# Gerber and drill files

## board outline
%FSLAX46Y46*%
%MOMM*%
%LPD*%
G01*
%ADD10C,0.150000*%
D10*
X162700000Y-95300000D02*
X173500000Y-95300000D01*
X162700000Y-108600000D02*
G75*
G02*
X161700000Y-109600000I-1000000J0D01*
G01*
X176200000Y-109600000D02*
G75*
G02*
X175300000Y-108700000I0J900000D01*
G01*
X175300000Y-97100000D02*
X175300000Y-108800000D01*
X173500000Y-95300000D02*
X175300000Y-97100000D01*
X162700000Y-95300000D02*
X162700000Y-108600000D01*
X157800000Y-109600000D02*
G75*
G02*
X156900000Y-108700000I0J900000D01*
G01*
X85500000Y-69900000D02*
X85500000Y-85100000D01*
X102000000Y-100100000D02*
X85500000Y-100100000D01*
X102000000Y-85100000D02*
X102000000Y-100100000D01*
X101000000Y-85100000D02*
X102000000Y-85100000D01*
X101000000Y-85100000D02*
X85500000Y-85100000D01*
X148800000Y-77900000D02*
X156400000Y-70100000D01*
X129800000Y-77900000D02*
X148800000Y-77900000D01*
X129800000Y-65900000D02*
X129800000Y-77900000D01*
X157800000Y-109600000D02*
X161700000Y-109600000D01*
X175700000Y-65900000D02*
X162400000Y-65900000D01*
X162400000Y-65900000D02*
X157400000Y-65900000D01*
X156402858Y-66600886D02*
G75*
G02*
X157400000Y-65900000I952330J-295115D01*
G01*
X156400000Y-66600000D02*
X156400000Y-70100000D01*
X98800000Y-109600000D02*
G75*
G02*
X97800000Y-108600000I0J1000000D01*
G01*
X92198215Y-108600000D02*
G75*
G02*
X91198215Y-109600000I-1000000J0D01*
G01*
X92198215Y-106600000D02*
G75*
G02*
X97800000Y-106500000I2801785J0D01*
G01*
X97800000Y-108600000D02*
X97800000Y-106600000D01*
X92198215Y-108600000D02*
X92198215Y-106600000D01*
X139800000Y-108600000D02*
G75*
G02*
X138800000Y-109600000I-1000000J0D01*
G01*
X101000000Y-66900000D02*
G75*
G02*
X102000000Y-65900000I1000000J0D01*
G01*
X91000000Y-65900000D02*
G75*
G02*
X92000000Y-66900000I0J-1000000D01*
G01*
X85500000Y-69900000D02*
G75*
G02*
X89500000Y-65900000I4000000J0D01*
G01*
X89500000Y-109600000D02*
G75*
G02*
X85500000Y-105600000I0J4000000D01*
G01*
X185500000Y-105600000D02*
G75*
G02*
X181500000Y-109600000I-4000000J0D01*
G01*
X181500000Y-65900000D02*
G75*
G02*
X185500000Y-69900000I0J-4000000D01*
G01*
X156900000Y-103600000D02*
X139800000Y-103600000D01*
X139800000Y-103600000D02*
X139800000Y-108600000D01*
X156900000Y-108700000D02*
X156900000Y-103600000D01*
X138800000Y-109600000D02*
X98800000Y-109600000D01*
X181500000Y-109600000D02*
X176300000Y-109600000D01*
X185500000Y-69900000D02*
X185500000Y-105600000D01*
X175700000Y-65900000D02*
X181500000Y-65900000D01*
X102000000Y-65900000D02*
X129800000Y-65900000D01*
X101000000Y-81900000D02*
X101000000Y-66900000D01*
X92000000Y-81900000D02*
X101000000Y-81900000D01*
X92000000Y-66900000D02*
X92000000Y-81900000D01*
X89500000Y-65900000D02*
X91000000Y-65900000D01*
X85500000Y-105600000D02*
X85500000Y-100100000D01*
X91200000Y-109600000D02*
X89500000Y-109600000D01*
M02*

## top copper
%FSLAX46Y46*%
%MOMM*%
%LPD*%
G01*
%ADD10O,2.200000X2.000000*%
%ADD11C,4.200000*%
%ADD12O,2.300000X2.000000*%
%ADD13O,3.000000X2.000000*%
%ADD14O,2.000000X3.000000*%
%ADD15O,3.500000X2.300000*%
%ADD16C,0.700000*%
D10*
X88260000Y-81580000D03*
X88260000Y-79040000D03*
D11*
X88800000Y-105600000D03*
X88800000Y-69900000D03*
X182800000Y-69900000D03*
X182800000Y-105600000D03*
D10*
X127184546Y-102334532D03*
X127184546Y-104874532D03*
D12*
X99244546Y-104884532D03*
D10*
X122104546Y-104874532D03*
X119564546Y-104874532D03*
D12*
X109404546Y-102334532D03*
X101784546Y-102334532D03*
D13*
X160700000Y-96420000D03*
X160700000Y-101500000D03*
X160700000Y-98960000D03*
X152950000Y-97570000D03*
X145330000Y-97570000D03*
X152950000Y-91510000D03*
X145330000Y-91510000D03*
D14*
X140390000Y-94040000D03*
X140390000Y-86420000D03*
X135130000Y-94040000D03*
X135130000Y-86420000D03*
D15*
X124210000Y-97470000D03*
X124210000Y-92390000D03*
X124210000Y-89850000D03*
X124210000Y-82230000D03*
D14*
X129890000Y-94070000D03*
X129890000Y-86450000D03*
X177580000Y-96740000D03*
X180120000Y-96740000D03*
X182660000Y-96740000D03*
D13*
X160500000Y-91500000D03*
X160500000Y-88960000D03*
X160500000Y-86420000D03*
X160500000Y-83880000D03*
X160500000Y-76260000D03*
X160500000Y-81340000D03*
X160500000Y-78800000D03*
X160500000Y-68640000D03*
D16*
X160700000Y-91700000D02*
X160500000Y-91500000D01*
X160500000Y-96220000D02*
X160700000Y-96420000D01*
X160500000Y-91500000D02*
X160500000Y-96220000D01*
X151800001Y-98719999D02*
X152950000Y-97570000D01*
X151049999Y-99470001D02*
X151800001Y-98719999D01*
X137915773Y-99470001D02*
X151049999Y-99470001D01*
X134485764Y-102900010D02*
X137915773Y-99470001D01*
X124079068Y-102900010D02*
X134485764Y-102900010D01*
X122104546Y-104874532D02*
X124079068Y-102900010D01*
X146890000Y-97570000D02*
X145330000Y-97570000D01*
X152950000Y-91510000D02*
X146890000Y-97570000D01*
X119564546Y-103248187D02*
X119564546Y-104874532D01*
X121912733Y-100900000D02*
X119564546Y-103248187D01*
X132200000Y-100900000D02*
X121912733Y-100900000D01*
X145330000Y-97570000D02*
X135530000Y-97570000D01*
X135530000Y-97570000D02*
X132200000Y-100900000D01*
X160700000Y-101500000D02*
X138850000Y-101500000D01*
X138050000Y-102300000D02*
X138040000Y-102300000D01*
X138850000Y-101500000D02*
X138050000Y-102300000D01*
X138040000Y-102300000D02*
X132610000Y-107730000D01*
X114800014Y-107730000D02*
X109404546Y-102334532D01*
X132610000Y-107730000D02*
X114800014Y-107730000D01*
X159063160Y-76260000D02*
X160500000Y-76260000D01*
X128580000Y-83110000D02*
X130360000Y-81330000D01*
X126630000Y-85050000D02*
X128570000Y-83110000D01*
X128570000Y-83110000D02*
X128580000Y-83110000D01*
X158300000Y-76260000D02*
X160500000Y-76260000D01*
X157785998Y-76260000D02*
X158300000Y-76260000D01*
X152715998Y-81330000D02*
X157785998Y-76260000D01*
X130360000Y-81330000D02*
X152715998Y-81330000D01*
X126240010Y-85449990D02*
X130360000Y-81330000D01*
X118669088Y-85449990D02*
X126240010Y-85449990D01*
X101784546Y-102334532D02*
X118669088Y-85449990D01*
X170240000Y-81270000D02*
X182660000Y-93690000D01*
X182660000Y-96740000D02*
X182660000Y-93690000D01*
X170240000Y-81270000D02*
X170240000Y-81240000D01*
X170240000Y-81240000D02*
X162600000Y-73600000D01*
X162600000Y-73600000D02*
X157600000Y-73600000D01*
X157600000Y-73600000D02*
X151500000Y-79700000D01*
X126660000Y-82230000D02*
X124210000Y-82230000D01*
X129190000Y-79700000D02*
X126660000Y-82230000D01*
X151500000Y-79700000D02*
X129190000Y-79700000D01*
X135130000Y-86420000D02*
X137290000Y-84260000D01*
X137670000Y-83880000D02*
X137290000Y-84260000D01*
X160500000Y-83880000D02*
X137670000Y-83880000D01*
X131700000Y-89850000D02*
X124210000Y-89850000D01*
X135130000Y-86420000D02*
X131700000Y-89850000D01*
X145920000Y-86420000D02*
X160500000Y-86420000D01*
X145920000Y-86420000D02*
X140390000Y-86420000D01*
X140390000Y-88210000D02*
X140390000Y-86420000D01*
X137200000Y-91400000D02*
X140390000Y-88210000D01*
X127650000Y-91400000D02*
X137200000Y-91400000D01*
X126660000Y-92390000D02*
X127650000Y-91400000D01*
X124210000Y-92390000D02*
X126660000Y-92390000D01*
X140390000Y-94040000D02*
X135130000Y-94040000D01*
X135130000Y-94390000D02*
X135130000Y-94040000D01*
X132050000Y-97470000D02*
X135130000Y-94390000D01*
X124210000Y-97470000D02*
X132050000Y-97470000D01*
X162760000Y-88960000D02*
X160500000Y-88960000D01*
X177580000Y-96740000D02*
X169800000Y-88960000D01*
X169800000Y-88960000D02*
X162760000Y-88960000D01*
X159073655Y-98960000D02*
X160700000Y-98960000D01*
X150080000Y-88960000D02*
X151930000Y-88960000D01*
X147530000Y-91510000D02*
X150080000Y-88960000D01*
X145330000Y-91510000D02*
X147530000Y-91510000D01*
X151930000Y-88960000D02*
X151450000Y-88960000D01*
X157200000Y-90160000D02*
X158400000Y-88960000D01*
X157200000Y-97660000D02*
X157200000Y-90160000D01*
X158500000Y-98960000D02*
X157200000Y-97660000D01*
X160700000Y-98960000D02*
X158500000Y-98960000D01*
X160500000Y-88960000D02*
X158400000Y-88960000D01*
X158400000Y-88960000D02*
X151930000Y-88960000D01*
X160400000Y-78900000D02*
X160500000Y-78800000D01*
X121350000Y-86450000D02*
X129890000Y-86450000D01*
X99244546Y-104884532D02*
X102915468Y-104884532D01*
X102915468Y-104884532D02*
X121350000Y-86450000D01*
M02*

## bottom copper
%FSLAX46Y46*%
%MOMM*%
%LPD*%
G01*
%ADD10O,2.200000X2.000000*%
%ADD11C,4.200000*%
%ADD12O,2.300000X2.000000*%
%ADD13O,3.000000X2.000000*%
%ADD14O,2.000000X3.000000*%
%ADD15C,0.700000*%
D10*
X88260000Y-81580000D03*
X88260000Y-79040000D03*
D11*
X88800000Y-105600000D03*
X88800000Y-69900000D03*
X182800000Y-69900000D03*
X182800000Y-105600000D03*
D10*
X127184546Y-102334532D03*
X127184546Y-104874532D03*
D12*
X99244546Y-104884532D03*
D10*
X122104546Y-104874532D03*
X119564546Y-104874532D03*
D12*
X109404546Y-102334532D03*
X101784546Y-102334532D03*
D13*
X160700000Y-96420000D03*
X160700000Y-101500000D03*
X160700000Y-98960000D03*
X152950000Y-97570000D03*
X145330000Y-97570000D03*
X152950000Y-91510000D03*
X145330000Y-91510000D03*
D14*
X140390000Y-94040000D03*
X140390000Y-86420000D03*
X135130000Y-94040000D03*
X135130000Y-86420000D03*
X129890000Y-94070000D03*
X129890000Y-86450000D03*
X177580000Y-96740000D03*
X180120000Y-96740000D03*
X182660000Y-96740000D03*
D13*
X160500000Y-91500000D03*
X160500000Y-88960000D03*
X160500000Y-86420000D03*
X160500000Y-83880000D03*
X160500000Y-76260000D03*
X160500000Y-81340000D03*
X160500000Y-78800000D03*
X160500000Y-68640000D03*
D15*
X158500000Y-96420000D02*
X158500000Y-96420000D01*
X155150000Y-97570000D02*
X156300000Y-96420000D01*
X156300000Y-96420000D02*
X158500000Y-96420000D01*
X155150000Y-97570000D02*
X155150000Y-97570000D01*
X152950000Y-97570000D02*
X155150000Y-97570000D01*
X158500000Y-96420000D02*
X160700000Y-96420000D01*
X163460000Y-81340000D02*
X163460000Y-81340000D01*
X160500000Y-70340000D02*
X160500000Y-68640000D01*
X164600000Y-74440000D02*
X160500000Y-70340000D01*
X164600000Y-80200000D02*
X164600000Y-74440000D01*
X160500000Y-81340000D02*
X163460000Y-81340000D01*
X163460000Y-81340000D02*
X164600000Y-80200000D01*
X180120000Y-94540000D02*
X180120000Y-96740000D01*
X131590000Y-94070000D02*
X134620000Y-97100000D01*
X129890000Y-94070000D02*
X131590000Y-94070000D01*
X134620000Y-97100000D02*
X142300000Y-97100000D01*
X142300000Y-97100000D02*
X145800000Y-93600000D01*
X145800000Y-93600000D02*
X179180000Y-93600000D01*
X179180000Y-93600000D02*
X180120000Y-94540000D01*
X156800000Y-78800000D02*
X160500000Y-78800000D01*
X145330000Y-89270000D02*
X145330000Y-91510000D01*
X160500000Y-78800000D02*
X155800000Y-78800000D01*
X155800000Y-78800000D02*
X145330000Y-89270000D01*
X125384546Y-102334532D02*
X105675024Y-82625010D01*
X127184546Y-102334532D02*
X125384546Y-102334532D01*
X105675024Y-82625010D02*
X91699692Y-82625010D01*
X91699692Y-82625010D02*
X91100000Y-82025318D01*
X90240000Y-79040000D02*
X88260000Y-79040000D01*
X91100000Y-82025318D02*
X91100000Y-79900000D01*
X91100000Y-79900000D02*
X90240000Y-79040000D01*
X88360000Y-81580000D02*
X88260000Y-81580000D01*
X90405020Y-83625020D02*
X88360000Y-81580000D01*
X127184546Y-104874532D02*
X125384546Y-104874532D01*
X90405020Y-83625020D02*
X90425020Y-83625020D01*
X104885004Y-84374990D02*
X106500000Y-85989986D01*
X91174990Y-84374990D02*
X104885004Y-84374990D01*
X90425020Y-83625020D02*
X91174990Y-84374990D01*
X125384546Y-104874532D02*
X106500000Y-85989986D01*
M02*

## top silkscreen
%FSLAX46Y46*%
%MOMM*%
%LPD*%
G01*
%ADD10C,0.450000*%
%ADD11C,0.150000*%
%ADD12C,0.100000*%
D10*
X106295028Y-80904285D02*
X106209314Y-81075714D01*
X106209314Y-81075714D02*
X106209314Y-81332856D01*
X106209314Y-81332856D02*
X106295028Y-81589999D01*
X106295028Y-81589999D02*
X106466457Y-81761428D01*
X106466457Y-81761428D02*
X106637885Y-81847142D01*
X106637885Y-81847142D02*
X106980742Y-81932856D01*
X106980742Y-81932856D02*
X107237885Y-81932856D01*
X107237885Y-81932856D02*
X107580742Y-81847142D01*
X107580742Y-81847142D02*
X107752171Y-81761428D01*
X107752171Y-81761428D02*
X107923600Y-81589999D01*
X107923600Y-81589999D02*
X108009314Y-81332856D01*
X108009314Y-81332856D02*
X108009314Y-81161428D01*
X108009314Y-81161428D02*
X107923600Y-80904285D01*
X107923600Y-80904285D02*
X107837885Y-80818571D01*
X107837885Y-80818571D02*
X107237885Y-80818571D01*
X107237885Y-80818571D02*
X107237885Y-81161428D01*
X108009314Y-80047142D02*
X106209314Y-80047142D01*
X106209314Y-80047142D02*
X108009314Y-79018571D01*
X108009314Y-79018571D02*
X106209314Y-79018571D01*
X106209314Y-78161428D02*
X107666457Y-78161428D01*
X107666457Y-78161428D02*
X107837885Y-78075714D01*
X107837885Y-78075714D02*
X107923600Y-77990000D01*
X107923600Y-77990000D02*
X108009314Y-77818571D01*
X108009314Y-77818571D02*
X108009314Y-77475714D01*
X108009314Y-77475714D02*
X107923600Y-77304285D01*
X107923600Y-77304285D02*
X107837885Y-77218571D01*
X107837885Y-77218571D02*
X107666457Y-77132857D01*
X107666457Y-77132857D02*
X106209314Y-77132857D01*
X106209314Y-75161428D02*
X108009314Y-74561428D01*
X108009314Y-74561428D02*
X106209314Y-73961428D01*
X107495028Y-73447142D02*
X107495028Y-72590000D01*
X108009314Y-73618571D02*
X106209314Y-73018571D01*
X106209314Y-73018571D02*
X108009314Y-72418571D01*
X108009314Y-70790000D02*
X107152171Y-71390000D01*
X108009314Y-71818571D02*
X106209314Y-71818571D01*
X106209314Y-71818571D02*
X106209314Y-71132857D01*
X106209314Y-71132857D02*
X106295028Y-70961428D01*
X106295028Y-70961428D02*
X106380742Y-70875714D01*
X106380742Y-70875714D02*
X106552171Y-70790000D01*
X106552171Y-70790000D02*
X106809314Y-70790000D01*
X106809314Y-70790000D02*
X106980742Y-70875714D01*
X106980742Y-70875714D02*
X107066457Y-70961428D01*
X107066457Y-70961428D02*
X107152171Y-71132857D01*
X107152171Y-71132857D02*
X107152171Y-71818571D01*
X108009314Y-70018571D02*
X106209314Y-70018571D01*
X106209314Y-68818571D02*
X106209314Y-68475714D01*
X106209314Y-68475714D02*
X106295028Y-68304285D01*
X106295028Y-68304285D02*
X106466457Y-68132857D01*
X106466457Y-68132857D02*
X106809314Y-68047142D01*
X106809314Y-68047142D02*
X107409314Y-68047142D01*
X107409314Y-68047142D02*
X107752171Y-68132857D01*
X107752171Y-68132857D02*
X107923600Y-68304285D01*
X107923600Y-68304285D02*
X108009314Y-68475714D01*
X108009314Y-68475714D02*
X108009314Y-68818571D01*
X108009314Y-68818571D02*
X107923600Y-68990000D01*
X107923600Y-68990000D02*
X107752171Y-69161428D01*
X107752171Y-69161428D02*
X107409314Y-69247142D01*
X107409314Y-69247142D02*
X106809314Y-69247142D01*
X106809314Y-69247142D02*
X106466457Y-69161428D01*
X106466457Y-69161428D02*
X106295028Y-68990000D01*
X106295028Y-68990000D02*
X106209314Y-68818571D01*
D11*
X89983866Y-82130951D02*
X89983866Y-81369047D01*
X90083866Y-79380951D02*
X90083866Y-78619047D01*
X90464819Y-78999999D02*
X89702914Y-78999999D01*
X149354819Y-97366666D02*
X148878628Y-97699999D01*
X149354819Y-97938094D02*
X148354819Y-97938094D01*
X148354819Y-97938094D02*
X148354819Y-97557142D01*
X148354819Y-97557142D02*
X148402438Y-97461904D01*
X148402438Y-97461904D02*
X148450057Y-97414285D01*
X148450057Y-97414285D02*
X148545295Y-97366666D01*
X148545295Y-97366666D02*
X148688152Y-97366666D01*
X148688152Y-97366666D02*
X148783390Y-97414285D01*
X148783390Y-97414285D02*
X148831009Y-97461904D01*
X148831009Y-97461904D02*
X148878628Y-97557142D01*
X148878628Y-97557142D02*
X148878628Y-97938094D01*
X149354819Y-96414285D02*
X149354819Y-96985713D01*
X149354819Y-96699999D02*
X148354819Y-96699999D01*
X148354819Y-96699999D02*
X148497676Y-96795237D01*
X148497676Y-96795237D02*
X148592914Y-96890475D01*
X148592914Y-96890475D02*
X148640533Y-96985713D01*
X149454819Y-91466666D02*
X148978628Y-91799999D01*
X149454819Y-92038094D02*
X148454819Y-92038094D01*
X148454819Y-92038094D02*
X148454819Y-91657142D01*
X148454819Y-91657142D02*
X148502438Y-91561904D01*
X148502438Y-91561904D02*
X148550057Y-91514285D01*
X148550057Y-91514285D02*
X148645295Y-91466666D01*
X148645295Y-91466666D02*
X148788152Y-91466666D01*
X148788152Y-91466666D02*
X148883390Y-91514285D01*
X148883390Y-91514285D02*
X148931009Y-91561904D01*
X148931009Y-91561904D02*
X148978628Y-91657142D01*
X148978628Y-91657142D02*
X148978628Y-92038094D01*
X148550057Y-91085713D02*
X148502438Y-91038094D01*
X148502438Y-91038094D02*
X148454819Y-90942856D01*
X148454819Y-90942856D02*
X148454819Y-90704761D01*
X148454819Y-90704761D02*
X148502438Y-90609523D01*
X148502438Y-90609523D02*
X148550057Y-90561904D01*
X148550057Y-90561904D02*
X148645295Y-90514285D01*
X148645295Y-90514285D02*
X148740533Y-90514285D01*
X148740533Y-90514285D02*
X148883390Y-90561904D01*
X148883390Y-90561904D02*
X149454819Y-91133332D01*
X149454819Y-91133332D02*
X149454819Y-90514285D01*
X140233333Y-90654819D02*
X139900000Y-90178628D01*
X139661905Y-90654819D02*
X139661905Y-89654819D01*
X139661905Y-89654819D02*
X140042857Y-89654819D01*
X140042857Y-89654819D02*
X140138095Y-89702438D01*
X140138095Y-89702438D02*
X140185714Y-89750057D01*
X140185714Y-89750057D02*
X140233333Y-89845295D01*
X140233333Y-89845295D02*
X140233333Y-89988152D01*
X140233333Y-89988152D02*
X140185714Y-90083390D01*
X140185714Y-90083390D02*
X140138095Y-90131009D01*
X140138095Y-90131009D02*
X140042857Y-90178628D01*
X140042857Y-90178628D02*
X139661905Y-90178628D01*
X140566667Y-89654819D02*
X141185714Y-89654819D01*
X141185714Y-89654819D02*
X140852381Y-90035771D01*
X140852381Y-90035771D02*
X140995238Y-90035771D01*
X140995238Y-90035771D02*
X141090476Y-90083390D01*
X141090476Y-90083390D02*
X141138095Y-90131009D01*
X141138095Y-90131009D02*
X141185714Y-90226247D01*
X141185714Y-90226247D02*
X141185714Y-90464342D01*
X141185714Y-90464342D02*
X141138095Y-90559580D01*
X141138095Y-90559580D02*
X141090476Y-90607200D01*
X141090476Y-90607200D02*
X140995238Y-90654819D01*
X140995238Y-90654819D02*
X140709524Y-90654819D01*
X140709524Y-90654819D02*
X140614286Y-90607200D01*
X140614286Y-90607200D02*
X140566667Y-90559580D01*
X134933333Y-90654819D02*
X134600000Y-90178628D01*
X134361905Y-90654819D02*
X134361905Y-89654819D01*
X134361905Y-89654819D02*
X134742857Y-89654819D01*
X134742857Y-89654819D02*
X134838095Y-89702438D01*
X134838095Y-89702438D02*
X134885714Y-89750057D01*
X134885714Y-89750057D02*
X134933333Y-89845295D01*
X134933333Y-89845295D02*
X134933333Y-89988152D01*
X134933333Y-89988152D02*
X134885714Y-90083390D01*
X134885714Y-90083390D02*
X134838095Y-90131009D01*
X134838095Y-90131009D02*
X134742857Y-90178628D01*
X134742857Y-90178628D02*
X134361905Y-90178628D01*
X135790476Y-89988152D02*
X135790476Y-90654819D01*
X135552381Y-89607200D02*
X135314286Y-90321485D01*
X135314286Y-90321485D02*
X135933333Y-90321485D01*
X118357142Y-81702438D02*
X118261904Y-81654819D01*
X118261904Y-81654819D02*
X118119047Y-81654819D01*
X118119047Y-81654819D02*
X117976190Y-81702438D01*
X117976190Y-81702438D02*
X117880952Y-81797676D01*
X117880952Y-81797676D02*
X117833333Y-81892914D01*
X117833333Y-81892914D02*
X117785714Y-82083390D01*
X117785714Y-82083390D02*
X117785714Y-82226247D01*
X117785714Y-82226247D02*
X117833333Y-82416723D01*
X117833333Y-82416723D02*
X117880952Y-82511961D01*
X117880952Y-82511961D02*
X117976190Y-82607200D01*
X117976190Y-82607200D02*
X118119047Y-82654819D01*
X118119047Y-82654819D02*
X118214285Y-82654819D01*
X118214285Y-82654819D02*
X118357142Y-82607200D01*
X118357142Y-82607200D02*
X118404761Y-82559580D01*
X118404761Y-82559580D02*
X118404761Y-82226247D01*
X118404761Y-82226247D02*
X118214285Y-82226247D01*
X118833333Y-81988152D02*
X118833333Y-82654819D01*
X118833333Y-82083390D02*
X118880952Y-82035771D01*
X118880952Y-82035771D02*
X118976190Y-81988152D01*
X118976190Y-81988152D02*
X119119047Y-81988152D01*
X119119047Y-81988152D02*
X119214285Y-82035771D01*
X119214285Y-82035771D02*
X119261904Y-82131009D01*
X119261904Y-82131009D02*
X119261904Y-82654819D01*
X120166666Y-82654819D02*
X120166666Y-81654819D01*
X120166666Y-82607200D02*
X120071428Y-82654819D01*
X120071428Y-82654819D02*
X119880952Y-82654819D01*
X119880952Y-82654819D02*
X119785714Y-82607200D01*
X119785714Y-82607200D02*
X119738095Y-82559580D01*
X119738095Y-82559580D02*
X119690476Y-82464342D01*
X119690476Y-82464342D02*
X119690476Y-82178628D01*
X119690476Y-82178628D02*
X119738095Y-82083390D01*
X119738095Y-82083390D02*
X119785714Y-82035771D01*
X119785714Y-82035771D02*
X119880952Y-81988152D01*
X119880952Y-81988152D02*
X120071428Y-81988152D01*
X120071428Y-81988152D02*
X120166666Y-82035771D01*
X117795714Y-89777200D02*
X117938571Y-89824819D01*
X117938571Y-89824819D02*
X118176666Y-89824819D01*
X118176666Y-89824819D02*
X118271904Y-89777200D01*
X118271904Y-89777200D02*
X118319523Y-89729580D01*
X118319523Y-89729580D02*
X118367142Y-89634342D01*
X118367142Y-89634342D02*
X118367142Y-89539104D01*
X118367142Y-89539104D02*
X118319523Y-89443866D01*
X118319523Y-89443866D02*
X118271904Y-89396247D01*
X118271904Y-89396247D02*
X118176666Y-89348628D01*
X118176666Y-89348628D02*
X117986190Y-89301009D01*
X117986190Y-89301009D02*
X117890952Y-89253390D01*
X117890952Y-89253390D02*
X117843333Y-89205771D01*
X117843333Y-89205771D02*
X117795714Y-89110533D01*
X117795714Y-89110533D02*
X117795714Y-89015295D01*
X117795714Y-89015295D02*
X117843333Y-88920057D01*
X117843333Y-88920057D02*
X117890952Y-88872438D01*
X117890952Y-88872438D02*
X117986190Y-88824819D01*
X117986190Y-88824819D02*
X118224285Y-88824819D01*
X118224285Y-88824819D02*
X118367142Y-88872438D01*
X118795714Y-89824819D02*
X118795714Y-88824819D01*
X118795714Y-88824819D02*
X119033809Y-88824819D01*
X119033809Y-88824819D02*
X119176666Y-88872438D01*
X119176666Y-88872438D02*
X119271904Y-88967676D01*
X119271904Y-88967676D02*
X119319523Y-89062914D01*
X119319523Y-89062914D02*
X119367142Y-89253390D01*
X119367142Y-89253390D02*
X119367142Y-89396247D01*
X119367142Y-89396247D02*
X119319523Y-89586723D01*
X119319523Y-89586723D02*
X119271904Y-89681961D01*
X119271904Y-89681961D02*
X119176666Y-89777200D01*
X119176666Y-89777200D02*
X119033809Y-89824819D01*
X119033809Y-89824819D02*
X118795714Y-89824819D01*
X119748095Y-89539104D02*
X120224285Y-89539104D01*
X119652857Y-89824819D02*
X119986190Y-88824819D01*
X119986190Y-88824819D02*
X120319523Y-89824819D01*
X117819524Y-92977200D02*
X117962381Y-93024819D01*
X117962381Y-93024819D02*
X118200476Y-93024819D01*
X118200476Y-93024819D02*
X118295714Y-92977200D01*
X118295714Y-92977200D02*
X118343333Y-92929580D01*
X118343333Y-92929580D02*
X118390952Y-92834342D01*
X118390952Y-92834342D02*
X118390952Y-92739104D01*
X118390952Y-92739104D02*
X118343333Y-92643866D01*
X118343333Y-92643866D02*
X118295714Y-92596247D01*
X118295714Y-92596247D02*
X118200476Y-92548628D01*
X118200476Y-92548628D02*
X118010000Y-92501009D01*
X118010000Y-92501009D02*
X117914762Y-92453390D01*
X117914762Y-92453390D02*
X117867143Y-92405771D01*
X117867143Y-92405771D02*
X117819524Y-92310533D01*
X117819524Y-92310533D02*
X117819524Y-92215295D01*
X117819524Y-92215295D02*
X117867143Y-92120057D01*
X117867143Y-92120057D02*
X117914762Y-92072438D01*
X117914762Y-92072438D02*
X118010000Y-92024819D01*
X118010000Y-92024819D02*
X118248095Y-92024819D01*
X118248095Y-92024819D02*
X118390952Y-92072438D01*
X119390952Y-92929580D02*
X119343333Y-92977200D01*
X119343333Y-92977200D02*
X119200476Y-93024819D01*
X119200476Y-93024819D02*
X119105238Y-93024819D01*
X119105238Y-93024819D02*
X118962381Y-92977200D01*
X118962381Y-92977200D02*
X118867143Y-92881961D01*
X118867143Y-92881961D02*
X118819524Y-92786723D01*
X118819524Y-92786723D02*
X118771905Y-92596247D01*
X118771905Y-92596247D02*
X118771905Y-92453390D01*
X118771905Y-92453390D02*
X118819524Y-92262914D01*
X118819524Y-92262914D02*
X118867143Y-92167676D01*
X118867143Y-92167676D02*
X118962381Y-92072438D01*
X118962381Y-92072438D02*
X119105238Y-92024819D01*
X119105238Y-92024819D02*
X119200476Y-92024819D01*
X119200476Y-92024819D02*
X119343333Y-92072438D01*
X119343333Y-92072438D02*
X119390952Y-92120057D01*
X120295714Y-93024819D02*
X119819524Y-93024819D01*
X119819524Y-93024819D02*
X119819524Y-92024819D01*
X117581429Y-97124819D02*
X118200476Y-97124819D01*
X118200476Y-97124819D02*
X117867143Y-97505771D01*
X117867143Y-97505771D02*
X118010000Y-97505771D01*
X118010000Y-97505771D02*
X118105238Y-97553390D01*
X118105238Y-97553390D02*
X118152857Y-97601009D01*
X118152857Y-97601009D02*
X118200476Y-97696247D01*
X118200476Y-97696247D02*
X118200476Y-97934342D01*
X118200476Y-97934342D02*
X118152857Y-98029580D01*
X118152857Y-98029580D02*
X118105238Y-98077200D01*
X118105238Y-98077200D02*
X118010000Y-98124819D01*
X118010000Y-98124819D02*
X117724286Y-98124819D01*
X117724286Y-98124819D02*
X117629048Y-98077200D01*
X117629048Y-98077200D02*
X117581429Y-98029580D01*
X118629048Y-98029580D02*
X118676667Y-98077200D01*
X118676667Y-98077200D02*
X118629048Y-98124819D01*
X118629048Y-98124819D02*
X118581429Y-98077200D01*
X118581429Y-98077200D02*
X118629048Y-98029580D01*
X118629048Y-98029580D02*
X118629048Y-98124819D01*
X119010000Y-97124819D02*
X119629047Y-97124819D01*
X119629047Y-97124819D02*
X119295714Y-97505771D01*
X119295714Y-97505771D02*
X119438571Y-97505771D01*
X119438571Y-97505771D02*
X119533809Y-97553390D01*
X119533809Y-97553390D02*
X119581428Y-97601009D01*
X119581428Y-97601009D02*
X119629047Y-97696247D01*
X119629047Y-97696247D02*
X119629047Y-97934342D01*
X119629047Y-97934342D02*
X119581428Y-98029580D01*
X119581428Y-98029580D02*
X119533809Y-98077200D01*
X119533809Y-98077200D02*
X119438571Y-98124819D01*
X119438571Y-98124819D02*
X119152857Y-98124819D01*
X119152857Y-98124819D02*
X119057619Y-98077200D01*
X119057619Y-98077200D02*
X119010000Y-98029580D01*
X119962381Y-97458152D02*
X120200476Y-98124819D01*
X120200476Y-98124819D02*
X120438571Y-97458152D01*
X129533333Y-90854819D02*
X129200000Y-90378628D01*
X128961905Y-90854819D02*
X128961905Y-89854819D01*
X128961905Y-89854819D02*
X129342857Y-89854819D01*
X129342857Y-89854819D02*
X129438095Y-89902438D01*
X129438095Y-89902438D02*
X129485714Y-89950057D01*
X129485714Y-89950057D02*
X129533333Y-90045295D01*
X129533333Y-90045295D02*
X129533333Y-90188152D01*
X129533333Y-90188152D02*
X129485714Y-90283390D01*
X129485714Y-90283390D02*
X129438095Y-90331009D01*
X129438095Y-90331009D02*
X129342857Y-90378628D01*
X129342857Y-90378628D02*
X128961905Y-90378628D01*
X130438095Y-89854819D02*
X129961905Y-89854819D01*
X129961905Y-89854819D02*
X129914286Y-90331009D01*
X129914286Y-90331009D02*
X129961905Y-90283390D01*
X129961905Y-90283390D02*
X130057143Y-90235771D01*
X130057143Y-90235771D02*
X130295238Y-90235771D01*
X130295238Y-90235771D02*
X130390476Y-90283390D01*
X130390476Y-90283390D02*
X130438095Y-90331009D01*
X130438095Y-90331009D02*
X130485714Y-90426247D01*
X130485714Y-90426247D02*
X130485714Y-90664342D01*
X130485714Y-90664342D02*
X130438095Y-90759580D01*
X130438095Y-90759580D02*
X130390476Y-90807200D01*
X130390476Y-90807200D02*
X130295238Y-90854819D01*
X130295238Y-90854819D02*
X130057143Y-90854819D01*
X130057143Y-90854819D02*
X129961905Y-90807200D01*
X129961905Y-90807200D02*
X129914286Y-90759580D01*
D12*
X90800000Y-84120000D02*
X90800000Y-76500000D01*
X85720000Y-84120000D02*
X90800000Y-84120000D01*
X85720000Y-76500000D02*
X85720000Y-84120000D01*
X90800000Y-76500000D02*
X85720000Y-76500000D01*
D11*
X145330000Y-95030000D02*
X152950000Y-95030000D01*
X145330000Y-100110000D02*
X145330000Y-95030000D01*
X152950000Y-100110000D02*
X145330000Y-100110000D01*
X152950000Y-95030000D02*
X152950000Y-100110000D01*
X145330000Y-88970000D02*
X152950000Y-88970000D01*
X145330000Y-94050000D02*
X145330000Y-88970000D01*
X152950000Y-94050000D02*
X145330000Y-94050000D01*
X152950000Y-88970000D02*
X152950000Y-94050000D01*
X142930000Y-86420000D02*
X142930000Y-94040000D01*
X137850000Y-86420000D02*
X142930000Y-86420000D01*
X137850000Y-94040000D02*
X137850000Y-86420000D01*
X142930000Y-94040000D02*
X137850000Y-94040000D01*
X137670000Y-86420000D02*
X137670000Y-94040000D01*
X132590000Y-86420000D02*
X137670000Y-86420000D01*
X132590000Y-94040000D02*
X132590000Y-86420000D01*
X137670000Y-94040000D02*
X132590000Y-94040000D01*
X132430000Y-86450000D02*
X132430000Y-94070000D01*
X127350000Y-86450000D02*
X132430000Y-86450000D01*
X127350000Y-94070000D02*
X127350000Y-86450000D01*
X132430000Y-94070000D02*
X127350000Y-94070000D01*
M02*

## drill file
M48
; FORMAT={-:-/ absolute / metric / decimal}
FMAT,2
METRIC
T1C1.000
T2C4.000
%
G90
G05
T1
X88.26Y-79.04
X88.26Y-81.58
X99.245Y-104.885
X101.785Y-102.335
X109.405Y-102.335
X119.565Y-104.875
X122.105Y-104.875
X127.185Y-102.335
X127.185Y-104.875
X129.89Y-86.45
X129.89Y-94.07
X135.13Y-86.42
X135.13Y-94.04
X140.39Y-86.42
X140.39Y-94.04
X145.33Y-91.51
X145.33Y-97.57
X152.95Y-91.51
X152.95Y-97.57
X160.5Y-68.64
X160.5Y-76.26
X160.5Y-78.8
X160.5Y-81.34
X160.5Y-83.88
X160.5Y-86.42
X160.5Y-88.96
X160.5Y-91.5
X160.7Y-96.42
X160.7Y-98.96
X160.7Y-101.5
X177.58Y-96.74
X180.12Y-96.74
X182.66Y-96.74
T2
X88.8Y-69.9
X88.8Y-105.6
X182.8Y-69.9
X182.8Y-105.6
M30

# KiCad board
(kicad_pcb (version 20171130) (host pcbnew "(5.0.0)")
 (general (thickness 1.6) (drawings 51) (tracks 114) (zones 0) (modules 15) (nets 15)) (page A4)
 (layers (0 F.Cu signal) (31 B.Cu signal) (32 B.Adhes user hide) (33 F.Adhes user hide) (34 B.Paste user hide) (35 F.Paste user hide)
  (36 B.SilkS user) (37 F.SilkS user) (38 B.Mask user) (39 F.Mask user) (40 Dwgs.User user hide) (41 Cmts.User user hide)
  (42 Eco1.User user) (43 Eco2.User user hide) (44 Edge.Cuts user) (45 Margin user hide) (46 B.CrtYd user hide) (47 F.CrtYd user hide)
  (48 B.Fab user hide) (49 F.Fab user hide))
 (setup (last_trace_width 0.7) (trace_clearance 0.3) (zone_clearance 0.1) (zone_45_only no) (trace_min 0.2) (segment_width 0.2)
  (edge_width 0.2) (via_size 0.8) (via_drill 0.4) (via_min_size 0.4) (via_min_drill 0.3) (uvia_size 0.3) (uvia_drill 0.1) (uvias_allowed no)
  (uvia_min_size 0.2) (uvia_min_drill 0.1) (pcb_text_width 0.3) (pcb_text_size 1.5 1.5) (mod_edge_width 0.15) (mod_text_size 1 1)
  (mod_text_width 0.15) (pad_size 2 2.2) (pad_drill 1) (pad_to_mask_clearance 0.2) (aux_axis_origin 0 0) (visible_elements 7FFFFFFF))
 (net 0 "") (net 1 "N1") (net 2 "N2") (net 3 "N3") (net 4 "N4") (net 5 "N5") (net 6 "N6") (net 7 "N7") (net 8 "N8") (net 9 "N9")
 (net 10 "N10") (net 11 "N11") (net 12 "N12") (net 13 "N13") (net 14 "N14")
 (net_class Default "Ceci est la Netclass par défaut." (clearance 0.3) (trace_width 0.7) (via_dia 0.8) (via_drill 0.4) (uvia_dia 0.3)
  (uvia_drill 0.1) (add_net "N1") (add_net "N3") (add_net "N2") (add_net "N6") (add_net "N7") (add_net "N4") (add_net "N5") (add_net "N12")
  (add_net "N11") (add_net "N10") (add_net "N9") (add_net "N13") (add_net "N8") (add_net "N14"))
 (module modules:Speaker (layer B.Cu) (at 90.8 76.5 270)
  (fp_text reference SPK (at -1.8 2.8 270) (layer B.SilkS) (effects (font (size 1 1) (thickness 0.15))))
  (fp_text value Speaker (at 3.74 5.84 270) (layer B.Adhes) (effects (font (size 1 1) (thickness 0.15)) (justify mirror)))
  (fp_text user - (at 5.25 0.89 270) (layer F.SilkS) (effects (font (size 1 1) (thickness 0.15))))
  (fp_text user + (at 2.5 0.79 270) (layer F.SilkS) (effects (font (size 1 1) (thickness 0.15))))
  (fp_line (start 7.62 0) (end 0 0) (layer F.SilkS) (width 0.1))
  (fp_line (start 7.62 5.08) (end 7.62 0) (layer F.SilkS) (width 0.1))
  (fp_line (start 0 5.08) (end 7.62 5.08) (layer F.SilkS) (width 0.1))
  (fp_line (start 0 0) (end 0 5.08) (layer F.SilkS) (width 0.1))
  (pad 2 thru_hole oval (at 5.08 2.54 270) (size 2 2.2) (drill 1) (layers *.Cu *.Paste *.Mask) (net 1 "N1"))
  (pad 1 thru_hole oval (at 2.54 2.54 270) (size 2 2.2) (drill 1) (layers *.Cu *.Paste *.Mask) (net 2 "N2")))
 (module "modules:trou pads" (layer F.Cu) (at 88.8 105.6)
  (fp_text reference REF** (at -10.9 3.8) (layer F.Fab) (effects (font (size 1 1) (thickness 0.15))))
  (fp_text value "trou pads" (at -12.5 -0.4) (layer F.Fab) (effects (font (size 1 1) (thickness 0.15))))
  (pad "" np_thru_hole circle (at 0 0) (size 4.2 4.2) (drill 4) (layers *.Cu *.Mask)))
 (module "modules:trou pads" (layer F.Cu) (at 88.8 69.9)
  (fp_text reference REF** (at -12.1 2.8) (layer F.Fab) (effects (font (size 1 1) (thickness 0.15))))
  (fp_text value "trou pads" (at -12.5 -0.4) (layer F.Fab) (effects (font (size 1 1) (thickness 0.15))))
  (pad "" np_thru_hole circle (at 0 0) (size 4.2 4.2) (drill 4) (layers *.Cu *.Mask)))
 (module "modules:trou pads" (layer F.Cu) (at 182.8 69.9)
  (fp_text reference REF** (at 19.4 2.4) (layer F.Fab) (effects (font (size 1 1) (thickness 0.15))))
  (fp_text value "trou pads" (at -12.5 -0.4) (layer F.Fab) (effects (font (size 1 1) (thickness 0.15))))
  (pad "" np_thru_hole circle (at 0 0) (size 4.2 4.2) (drill 4) (layers *.Cu *.Mask)))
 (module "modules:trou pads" (layer F.Cu) (at 182.8 105.6)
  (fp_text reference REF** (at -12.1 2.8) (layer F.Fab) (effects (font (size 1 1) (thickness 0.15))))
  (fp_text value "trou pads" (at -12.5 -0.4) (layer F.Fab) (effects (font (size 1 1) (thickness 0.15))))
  (pad "" np_thru_hole circle (at 0 0) (size 4.2 4.2) (drill 4) (layers *.Cu *.Mask)))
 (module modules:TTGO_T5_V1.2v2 (layer F.Cu) (at 127.734546 102.554532 90)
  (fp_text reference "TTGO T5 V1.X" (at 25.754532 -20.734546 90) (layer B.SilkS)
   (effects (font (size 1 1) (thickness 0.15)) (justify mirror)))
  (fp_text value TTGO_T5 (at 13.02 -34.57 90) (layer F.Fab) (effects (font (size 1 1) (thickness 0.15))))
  (pad "HP +" thru_hole oval (at 0.22 -0.55 90) (size 2 2.2) (drill 1) (layers *.Cu *.Paste *.Mask) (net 2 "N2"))
  (pad "HP -" thru_hole oval (at -2.32 -0.55 90) (size 2 2.2) (drill 1) (layers *.Cu *.Paste *.Mask) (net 1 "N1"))
  (pad 12 thru_hole oval (at -2.33 -28.49 90) (size 2 2.3) (drill 1) (layers *.Cu *.Paste *.Mask) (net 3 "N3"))
  (pad 3 thru_hole oval (at -2.32 -5.63 90) (size 2 2.2) (drill 1) (layers *.Cu *.Paste *.Mask) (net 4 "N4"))
  (pad 4 thru_hole oval (at -2.32 -8.17 90) (size 2 2.2) (drill 1) (layers *.Cu *.Paste *.Mask) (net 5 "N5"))
  (pad 20 thru_hole oval (at 0.22 -18.33 90) (size 2 2.3) (drill 1) (layers *.Cu *.Paste *.Mask) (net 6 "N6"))
  (pad 23 thru_hole oval (at 0.22 -25.95 90) (size 2 2.3) (drill 1) (layers *.Cu *.Paste *.Mask) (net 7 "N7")))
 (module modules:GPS (layer F.Cu) (at 160.7 96.42 270)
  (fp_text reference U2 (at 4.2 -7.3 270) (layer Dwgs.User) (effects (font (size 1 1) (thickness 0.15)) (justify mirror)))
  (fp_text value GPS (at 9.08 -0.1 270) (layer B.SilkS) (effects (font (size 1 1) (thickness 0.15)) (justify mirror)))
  (pad 1 thru_hole oval (at 0 0 270) (size 2 3) (drill 1) (layers *.Cu *.Paste *.Mask) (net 4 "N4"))
  (pad 3 thru_hole oval (at 5.08 0 270) (size 2 3) (drill 1) (layers *.Cu *.Paste *.Mask) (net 6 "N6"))
  (pad 2 thru_hole oval (at 2.54 0 270) (size 2 3) (drill 1) (layers *.Cu *.Paste *.Mask) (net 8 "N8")))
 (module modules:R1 (layer F.Cu) (at 145.33 97.57 270)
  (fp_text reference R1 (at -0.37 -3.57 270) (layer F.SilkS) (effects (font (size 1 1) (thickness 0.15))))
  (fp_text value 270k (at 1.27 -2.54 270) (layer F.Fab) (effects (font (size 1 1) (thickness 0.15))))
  (fp_line (start -2.54 0) (end -2.54 -7.62) (layer F.SilkS) (width 0.15))
  (fp_line (start 2.54 0) (end -2.54 0) (layer F.SilkS) (width 0.15))
  (fp_line (start 2.54 -7.62) (end 2.54 0) (layer F.SilkS) (width 0.15))
  (fp_line (start -2.54 -7.62) (end 2.54 -7.62) (layer F.SilkS) (width 0.15))
  (pad 2 thru_hole oval (at 0 -7.62 270) (size 2 3) (drill 1) (layers *.Cu *.Paste *.Mask) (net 4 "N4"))
  (pad 1 thru_hole oval (at 0 0 270) (size 2 3) (drill 1) (layers *.Cu *.Paste *.Mask) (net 5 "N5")))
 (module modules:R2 (layer F.Cu) (at 145.33 91.51 270)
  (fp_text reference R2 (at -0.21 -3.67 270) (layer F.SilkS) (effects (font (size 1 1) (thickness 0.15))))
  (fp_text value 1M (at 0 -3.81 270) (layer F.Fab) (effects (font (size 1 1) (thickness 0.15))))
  (fp_line (start -2.54 0) (end -2.54 -7.62) (layer F.SilkS) (width 0.15))
  (fp_line (start 2.54 0) (end -2.54 0) (layer F.SilkS) (width 0.15))
  (fp_line (start 2.54 -7.62) (end 2.54 0) (layer F.SilkS) (width 0.15))
  (fp_line (start -2.54 -7.62) (end 2.54 -7.62) (layer F.SilkS) (width 0.15))
  (pad 2 thru_hole oval (at 0 -7.62 270) (size 2 3) (drill 1) (layers *.Cu *.Paste *.Mask) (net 5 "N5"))
  (pad 1 thru_hole oval (at 0 0 270) (size 2 3) (drill 1) (layers *.Cu *.Paste *.Mask) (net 8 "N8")))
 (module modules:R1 (layer F.Cu) (at 140.39 86.42 180)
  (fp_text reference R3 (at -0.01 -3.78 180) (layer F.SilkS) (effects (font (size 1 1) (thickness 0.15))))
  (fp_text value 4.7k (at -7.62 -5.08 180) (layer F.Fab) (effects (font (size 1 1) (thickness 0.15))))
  (fp_line (start -2.54 0) (end -2.54 -7.62) (layer F.SilkS) (width 0.15))
  (fp_line (start 2.54 0) (end -2.54 0) (layer F.SilkS) (width 0.15))
  (fp_line (start 2.54 -7.62) (end 2.54 0) (layer F.SilkS) (width 0.15))
  (fp_line (start -2.54 -7.62) (end 2.54 -7.62) (layer F.SilkS) (width 0.15))
  (pad 2 thru_hole oval (at 0 -7.62 180) (size 2 3) (drill 1) (layers *.Cu *.Paste *.Mask) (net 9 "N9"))
  (pad 1 thru_hole oval (at 0 0 180) (size 2 3) (drill 1) (layers *.Cu *.Paste *.Mask) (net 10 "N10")))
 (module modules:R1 (layer F.Cu) (at 135.13 86.42 180)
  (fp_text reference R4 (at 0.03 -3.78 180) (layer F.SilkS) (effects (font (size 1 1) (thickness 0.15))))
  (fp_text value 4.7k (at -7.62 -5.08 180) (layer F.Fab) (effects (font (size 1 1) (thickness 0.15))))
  (fp_line (start -2.54 0) (end -2.54 -7.62) (layer F.SilkS) (width 0.15))
  (fp_line (start 2.54 0) (end -2.54 0) (layer F.SilkS) (width 0.15))
  (fp_line (start 2.54 -7.62) (end 2.54 0) (layer F.SilkS) (width 0.15))
  (fp_line (start -2.54 -7.62) (end 2.54 -7.62) (layer F.SilkS) (width 0.15))
  (pad 2 thru_hole oval (at 0 -7.62 180) (size 2 3) (drill 1) (layers *.Cu *.Paste *.Mask) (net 9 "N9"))
  (pad 1 thru_hole oval (at 0 0 180) (size 2 3) (drill 1) (layers *.Cu *.Paste *.Mask) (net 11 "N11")))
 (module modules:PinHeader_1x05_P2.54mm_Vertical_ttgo (layer F.Cu) (at 124.21 84.77)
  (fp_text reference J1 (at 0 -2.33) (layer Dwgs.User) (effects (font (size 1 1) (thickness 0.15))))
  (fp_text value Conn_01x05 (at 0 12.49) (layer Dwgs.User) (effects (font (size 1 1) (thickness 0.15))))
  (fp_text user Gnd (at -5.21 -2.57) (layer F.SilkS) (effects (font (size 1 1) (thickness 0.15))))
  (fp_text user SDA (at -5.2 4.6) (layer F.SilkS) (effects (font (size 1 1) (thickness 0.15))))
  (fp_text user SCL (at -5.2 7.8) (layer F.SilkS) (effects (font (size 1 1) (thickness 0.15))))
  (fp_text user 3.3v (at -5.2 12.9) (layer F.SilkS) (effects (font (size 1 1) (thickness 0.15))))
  (pad 5 smd oval (at 0 12.7) (size 3.5 2.3) (layers F.Cu F.Paste F.Mask) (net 9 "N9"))
  (pad 4 smd oval (at 0 7.62) (size 3.5 2.3) (layers F.Cu F.Paste F.Mask) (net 10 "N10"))
  (pad 3 smd oval (at 0 5.08) (size 3.5 2.3) (layers F.Cu F.Paste F.Mask) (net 11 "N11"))
  (pad 1 smd oval (at 0 -2.54) (size 3.5 2.3) (layers F.Cu F.Paste F.Mask) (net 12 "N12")))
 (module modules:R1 (layer F.Cu) (at 129.89 86.45 180)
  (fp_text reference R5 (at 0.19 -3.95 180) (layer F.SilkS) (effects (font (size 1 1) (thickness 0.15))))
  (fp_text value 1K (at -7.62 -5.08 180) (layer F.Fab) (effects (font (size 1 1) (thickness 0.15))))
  (fp_line (start -2.54 0) (end -2.54 -7.62) (layer F.SilkS) (width 0.15))
  (fp_line (start 2.54 0) (end -2.54 0) (layer F.SilkS) (width 0.15))
  (fp_line (start 2.54 -7.62) (end 2.54 0) (layer F.SilkS) (width 0.15))
  (fp_line (start -2.54 -7.62) (end 2.54 -7.62) (layer F.SilkS) (width 0.15))
  (pad 2 thru_hole oval (at 0 -7.62 180) (size 2 3) (drill 1) (layers *.Cu *.Paste *.Mask) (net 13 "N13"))
  (pad 1 thru_hole oval (at 0 0 180) (size 2 3) (drill 1) (layers *.Cu *.Paste *.Mask) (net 3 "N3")))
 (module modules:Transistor (layer F.Cu) (at 185.2 94.2 180)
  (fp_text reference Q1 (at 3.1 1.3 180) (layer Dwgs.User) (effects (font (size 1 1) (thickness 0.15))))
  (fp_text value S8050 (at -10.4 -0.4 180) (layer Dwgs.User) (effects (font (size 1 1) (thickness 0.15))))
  (pad 3 thru_hole oval (at 7.62 -2.54 180) (size 2 3) (drill 1) (layers *.Cu *.Paste *.Mask) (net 8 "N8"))
  (pad 2 thru_hole oval (at 5.08 -2.54 180) (size 2 3) (drill 1) (layers *.Cu *.Paste *.Mask) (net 13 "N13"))
  (pad 1 thru_hole oval (at 2.54 -2.54 180) (size 2 3) (drill 1) (layers *.Cu *.Paste *.Mask) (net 12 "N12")))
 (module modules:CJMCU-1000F (layer B.Cu) (at 163.04 78.8 270)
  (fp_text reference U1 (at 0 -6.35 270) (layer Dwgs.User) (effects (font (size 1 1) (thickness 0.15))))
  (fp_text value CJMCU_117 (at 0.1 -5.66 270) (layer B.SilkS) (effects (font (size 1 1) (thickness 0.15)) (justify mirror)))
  (pad 1 thru_hole oval (at 12.7 2.54 270) (size 2 3) (drill 1) (layers *.Cu *.Paste *.Mask) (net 4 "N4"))
  (pad 2 thru_hole oval (at 10.16 2.54 270) (size 2 3) (drill 1) (layers *.Cu *.Paste *.Mask) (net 8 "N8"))
  (pad 3 thru_hole oval (at 7.62 2.54 270) (size 2 3) (drill 1) (layers *.Cu *.Paste *.Mask) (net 10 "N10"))
  (pad 4 thru_hole oval (at 5.08 2.54 270) (size 2 3) (drill 1) (layers *.Cu *.Paste *.Mask) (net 11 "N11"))
  (pad 7 thru_hole oval (at -2.54 2.54 270) (size 2 3) (drill 1) (layers *.Cu *.Paste *.Mask) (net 7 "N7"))
  (pad 5 thru_hole oval (at 2.54 2.54 270) (size 2 3) (drill 1) (layers *.Cu *.Paste *.Mask) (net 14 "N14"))
  (pad 6 thru_hole oval (at 0 2.54 270) (size 2 3) (drill 1) (layers *.Cu *.Paste *.Mask) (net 8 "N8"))
  (pad 10 thru_hole oval (at -10.16 2.54 270) (size 2 3) (drill 1) (layers *.Cu *.Paste *.Mask) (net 14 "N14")))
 (gr_line (start 162.7 95.3) (end 173.5 95.3) (layer Edge.Cuts) (width 0.15))
 (gr_arc (start 161.7 108.6) (end 161.7 109.6) (angle -90) (layer Edge.Cuts) (width 0.15))
 (gr_arc (start 176.2 108.7) (end 175.3 108.7) (angle -90) (layer Edge.Cuts) (width 0.15))
 (gr_line (start 175.3 97.1) (end 175.3 108.8) (layer Edge.Cuts) (width 0.15))
 (gr_line (start 173.5 95.3) (end 175.3 97.1) (layer Edge.Cuts) (width 0.15))
 (gr_line (start 162.7 95.3) (end 162.7 108.6) (layer Edge.Cuts) (width 0.15))
 (gr_arc (start 157.8 108.7) (end 156.9 108.7) (angle -90) (layer Edge.Cuts) (width 0.15))
 (gr_line (start 85.5 69.9) (end 85.5 85.1) (layer Edge.Cuts) (width 0.15))
 (gr_line (start 102 100.1) (end 85.5 100.1) (layer Edge.Cuts) (width 0.15))
 (gr_line (start 102 85.1) (end 102 100.1) (layer Edge.Cuts) (width 0.15))
 (gr_line (start 101 85.1) (end 102 85.1) (layer Edge.Cuts) (width 0.15))
 (gr_line (start 101 85.1) (end 85.5 85.1) (layer Edge.Cuts) (width 0.15))
 (gr_line (start 148.8 77.9) (end 156.4 70.1) (layer Edge.Cuts) (width 0.15))
 (gr_line (start 129.8 77.9) (end 148.8 77.9) (layer Edge.Cuts) (width 0.15))
 (gr_line (start 129.8 65.9) (end 129.8 77.9) (layer Edge.Cuts) (width 0.15))
 (gr_line (start 157.8 109.6) (end 161.7 109.6) (layer Edge.Cuts) (width 0.15))
 (gr_line (start 175.7 65.9) (end 162.4 65.9) (layer Edge.Cuts) (width 0.15))
 (gr_line (start 162.4 65.9) (end 157.4 65.9) (layer Edge.Cuts) (width 0.15))
 (gr_arc (start 157.355188 66.896001) (end 157.4 65.9) (angle -75.35856355) (layer Edge.Cuts) (width 0.15))
 (gr_line (start 156.4 66.6) (end 156.4 70.1) (layer Edge.Cuts) (width 0.15))
 (gr_arc (start 98.8 108.6) (end 97.8 108.6) (angle -90) (layer Edge.Cuts) (width 0.15))
 (gr_arc (start 91.198215 108.6) (end 91.198215 109.6) (angle -90) (layer Edge.Cuts) (width 0.15))
 (gr_arc (start 95 106.6) (end 97.8 106.5) (angle -177.9545915) (layer Edge.Cuts) (width 0.15))
 (gr_line (start 97.8 108.6) (end 97.8 106.6) (layer Edge.Cuts) (width 0.15))
 (gr_line (start 92.198215 108.6) (end 92.198215 106.6) (layer Edge.Cuts) (width 0.15))
 (gr_arc (start 138.8 108.6) (end 138.8 109.6) (angle -90) (layer Edge.Cuts) (width 0.15))
 (gr_arc (start 102 66.9) (end 102 65.9) (angle -90) (layer Edge.Cuts) (width 0.15))
 (gr_arc (start 91 66.9) (end 92 66.9) (angle -90) (layer Edge.Cuts) (width 0.15))
 (gr_arc (start 89.5 69.9) (end 89.5 65.9) (angle -90) (layer Edge.Cuts) (width 0.15))
 (gr_arc (start 89.5 105.6) (end 85.5 105.6) (angle -90) (layer Edge.Cuts) (width 0.15))
 (gr_arc (start 181.5 105.6) (end 181.5 109.6) (angle -90) (layer Edge.Cuts) (width 0.15))
 (gr_arc (start 181.5 69.9) (end 185.5 69.9) (angle -90) (layer Edge.Cuts) (width 0.15))
 (gr_line (start 156.9 103.6) (end 139.8 103.6) (layer Edge.Cuts) (width 0.15))
 (gr_line (start 139.8 103.6) (end 139.8 108.6) (layer Edge.Cuts) (width 0.15))
 (gr_line (start 156.9 108.7) (end 156.9 103.6) (layer Edge.Cuts) (width 0.15))
 (gr_line (start 138.8 109.6) (end 98.8 109.6) (layer Edge.Cuts) (width 0.15))
 (gr_line (start 181.5 109.6) (end 176.3 109.6) (layer Edge.Cuts) (width 0.15))
 (gr_line (start 185.5 69.9) (end 185.5 105.6) (layer Edge.Cuts) (width 0.15))
 (gr_line (start 175.7 65.9) (end 181.5 65.9) (layer Edge.Cuts) (width 0.15))
 (gr_line (start 102 65.9) (end 129.8 65.9) (layer Edge.Cuts) (width 0.15))
 (gr_line (start 101 81.9) (end 101 66.9) (layer Edge.Cuts) (width 0.15))
 (gr_line (start 92 81.9) (end 101 81.9) (layer Edge.Cuts) (width 0.15))
 (gr_line (start 92 66.9) (end 92 81.9) (layer Edge.Cuts) (width 0.15))
 (gr_line (start 89.5 65.9) (end 91 65.9) (layer Edge.Cuts) (width 0.15))
 (gr_line (start 85.5 105.6) (end 85.5 100.1) (layer Edge.Cuts) (width 0.15))
 (gr_line (start 91.2 109.6) (end 89.5 109.6) (layer Edge.Cuts) (width 0.15))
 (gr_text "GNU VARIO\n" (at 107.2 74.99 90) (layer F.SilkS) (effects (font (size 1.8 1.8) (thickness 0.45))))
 (segment (start 160.7 91.7) (end 160.5 91.5) (width 0.7) (layer F.Cu) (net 4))
 (segment (start 160.5 96.22) (end 160.7 96.42) (width 0.7) (layer F.Cu) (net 4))
 (segment (start 160.5 91.5) (end 160.5 96.22) (width 0.7) (layer F.Cu) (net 4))
 (segment (start 151.800001 98.719999) (end 152.95 97.57) (width 0.7) (layer F.Cu) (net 4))
 (segment (start 151.049999 99.470001) (end 151.800001 98.719999) (width 0.7) (layer F.Cu) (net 4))
 (segment (start 137.915773 99.470001) (end 151.049999 99.470001) (width 0.7) (layer F.Cu) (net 4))
 (segment (start 134.485764 102.90001) (end 137.915773 99.470001) (width 0.7) (layer F.Cu) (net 4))
 (segment (start 124.079068 102.90001) (end 134.485764 102.90001) (width 0.7) (layer F.Cu) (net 4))
 (segment (start 122.104546 104.874532) (end 124.079068 102.90001) (width 0.7) (layer F.Cu) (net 4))
 (segment (start 158.5 96.42) (end 158.5 96.42) (width 0.7) (layer B.Cu) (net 4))
 (segment (start 155.15 97.57) (end 156.3 96.42) (width 0.7) (layer B.Cu) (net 4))
 (segment (start 156.3 96.42) (end 158.5 96.42) (width 0.7) (layer B.Cu) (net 4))
 (segment (start 155.15 97.57) (end 155.15 97.57) (width 0.7) (layer B.Cu) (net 4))
 (segment (start 152.95 97.57) (end 155.15 97.57) (width 0.7) (layer B.Cu) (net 4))
 (segment (start 158.5 96.42) (end 160.7 96.42) (width 0.7) (layer B.Cu) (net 4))
 (segment (start 146.89 97.57) (end 145.33 97.57) (width 0.7) (layer F.Cu) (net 5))
 (segment (start 152.95 91.51) (end 146.89 97.57) (width 0.7) (layer F.Cu) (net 5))
 (segment (start 119.564546 103.248187) (end 119.564546 104.874532) (width 0.7) (layer F.Cu) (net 5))
 (segment (start 121.912733 100.9) (end 119.564546 103.248187) (width 0.7) (layer F.Cu) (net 5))
 (segment (start 132.2 100.9) (end 121.912733 100.9) (width 0.7) (layer F.Cu) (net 5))
 (segment (start 145.33 97.57) (end 135.53 97.57) (width 0.7) (layer F.Cu) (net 5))
 (segment (start 135.53 97.57) (end 132.2 100.9) (width 0.7) (layer F.Cu) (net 5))
 (segment (start 160.7 101.5) (end 138.85 101.5) (width 0.7) (layer F.Cu) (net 6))
 (segment (start 138.05 102.3) (end 138.04 102.3) (width 0.7) (layer F.Cu) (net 6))
 (segment (start 138.85 101.5) (end 138.05 102.3) (width 0.7) (layer F.Cu) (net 6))
 (segment (start 138.04 102.3) (end 132.61 107.73) (width 0.7) (layer F.Cu) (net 6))
 (segment (start 114.800014 107.73) (end 109.404546 102.334532) (width 0.7) (layer F.Cu) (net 6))
 (segment (start 132.61 107.73) (end 114.800014 107.73) (width 0.7) (layer F.Cu) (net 6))
 (segment (start 159.06316 76.26) (end 160.5 76.26) (width 0.7) (layer F.Cu) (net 7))
 (segment (start 128.58 83.11) (end 130.36 81.33) (width 0.7) (layer F.Cu) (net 7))
 (segment (start 126.63 85.05) (end 128.57 83.11) (width 0.7) (layer F.Cu) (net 7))
 (segment (start 128.57 83.11) (end 128.58 83.11) (width 0.7) (layer F.Cu) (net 7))
 (segment (start 158.3 76.26) (end 160.5 76.26) (width 0.7) (layer F.Cu) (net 7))
 (segment (start 157.785998 76.26) (end 158.3 76.26) (width 0.7) (layer F.Cu) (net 7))
 (segment (start 152.715998 81.33) (end 157.785998 76.26) (width 0.7) (layer F.Cu) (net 7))
 (segment (start 130.36 81.33) (end 152.715998 81.33) (width 0.7) (layer F.Cu) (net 7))
 (segment (start 126.24001 85.44999) (end 130.36 81.33) (width 0.7) (layer F.Cu) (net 7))
 (segment (start 118.669088 85.44999) (end 126.24001 85.44999) (width 0.7) (layer F.Cu) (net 7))
 (segment (start 101.784546 102.334532) (end 118.669088 85.44999) (width 0.7) (layer F.Cu) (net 7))
 (segment (start 163.46 81.34) (end 163.46 81.34) (width 0.7) (layer B.Cu) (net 14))
 (segment (start 160.5 70.34) (end 160.5 68.64) (width 0.7) (layer B.Cu) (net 14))
 (segment (start 164.6 74.44) (end 160.5 70.34) (width 0.7) (layer B.Cu) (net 14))
 (segment (start 164.6 80.2) (end 164.6 74.44) (width 0.7) (layer B.Cu) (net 14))
 (segment (start 160.5 81.34) (end 163.46 81.34) (width 0.7) (layer B.Cu) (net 14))
 (segment (start 163.46 81.34) (end 164.6 80.2) (width 0.7) (layer B.Cu) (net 14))
 (segment (start 170.24 81.27) (end 182.66 93.69) (width 0.7) (layer F.Cu) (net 12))
 (segment (start 182.66 96.74) (end 182.66 93.69) (width 0.7) (layer F.Cu) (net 12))
 (segment (start 170.24 81.27) (end 170.24 81.24) (width 0.7) (layer F.Cu) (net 12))
 (segment (start 170.24 81.24) (end 162.6 73.6) (width 0.7) (layer F.Cu) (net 12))
 (segment (start 162.6 73.6) (end 157.6 73.6) (width 0.7) (layer F.Cu) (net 12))
 (segment (start 157.6 73.6) (end 151.5 79.7) (width 0.7) (layer F.Cu) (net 12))
 (segment (start 126.66 82.23) (end 124.21 82.23) (width 0.7) (layer F.Cu) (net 12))
 (segment (start 129.19 79.7) (end 126.66 82.23) (width 0.7) (layer F.Cu) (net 12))
 (segment (start 151.5 79.7) (end 129.19 79.7) (width 0.7) (layer F.Cu) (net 12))
 (segment (start 135.13 86.42) (end 137.29 84.26) (width 0.7) (layer F.Cu) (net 11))
 (segment (start 137.67 83.88) (end 137.29 84.26) (width 0.7) (layer F.Cu) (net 11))
 (segment (start 160.5 83.88) (end 137.67 83.88) (width 0.7) (layer F.Cu) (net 11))
 (segment (start 131.7 89.85) (end 124.21 89.85) (width 0.7) (layer F.Cu) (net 11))
 (segment (start 135.13 86.42) (end 131.7 89.85) (width 0.7) (layer F.Cu) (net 11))
 (segment (start 145.92 86.42) (end 160.5 86.42) (width 0.7) (layer F.Cu) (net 10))
 (segment (start 145.92 86.42) (end 140.39 86.42) (width 0.7) (layer F.Cu) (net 10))
 (segment (start 140.39 88.21) (end 140.39 86.42) (width 0.7) (layer F.Cu) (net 10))
 (segment (start 137.2 91.4) (end 140.39 88.21) (width 0.7) (layer F.Cu) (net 10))
 (segment (start 127.65 91.4) (end 137.2 91.4) (width 0.7) (layer F.Cu) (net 10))
 (segment (start 126.66 92.39) (end 127.65 91.4) (width 0.7) (layer F.Cu) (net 10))
 (segment (start 124.21 92.39) (end 126.66 92.39) (width 0.7) (layer F.Cu) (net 10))
 (segment (start 140.39 94.04) (end 135.13 94.04) (width 0.7) (layer F.Cu) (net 9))
 (segment (start 135.13 94.39) (end 135.13 94.04) (width 0.7) (layer F.Cu) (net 9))
 (segment (start 132.05 97.47) (end 135.13 94.39) (width 0.7) (layer F.Cu) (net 9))
 (segment (start 124.21 97.47) (end 132.05 97.47) (width 0.7) (layer F.Cu) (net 9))
 (segment (start 180.12 94.54) (end 180.12 96.74) (width 0.7) (layer B.Cu) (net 13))
 (segment (start 131.59 94.07) (end 134.62 97.1) (width 0.7) (layer B.Cu) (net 13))
 (segment (start 129.89 94.07) (end 131.59 94.07) (width 0.7) (layer B.Cu) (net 13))
 (segment (start 134.62 97.1) (end 142.3 97.1) (width 0.7) (layer B.Cu) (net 13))
 (segment (start 142.3 97.1) (end 145.8 93.6) (width 0.7) (layer B.Cu) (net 13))
 (segment (start 145.8 93.6) (end 179.18 93.6) (width 0.7) (layer B.Cu) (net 13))
 (segment (start 179.18 93.6) (end 180.12 94.54) (width 0.7) (layer B.Cu) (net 13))
 (segment (start 162.76 88.96) (end 160.5 88.96) (width 0.7) (layer F.Cu) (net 8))
 (segment (start 177.58 96.74) (end 169.8 88.96) (width 0.7) (layer F.Cu) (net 8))
 (segment (start 169.8 88.96) (end 162.76 88.96) (width 0.7) (layer F.Cu) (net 8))
 (segment (start 159.073655 98.96) (end 160.7 98.96) (width 0.7) (layer F.Cu) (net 8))
 (segment (start 150.08 88.96) (end 151.93 88.96) (width 0.7) (layer F.Cu) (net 8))
 (segment (start 147.53 91.51) (end 150.08 88.96) (width 0.7) (layer F.Cu) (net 8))
 (segment (start 145.33 91.51) (end 147.53 91.51) (width 0.7) (layer F.Cu) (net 8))
 (segment (start 151.93 88.96) (end 151.45 88.96) (width 0.7) (layer F.Cu) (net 8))
 (segment (start 157.2 90.16) (end 158.4 88.96) (width 0.7) (layer F.Cu) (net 8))
 (segment (start 157.2 97.66) (end 157.2 90.16) (width 0.7) (layer F.Cu) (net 8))
 (segment (start 158.5 98.96) (end 157.2 97.66) (width 0.7) (layer F.Cu) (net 8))
 (segment (start 160.7 98.96) (end 158.5 98.96) (width 0.7) (layer F.Cu) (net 8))
 (segment (start 160.5 88.96) (end 158.4 88.96) (width 0.7) (layer F.Cu) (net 8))
 (segment (start 158.4 88.96) (end 151.93 88.96) (width 0.7) (layer F.Cu) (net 8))
 (segment (start 160.4 78.9) (end 160.5 78.8) (width 0.7) (layer F.Cu) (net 8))
 (segment (start 156.8 78.8) (end 160.5 78.8) (width 0.7) (layer B.Cu) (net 8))
 (segment (start 145.33 89.27) (end 145.33 91.51) (width 0.7) (layer B.Cu) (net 8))
 (segment (start 160.5 78.8) (end 155.8 78.8) (width 0.7) (layer B.Cu) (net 8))
 (segment (start 155.8 78.8) (end 145.33 89.27) (width 0.7) (layer B.Cu) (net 8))
 (segment (start 121.35 86.45) (end 129.89 86.45) (width 0.7) (layer F.Cu) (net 3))
 (segment (start 99.244546 104.884532) (end 102.915468 104.884532) (width 0.7) (layer F.Cu) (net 3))
 (segment (start 102.915468 104.884532) (end 121.35 86.45) (width 0.7) (layer F.Cu) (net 3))
 (segment (start 125.384546 102.334532) (end 105.675024 82.62501) (width 0.7) (layer B.Cu) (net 2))
 (segment (start 127.184546 102.334532) (end 125.384546 102.334532) (width 0.7) (layer B.Cu) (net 2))
 (segment (start 105.675024 82.62501) (end 91.699692 82.62501) (width 0.7) (layer B.Cu) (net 2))
 (segment (start 91.699692 82.62501) (end 91.1 82.025318) (width 0.7) (layer B.Cu) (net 2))
 (segment (start 90.24 79.04) (end 88.26 79.04) (width 0.7) (layer B.Cu) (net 2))
 (segment (start 91.1 82.025318) (end 91.1 79.9) (width 0.7) (layer B.Cu) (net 2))
 (segment (start 91.1 79.9) (end 90.24 79.04) (width 0.7) (layer B.Cu) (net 2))
 (segment (start 88.36 81.58) (end 88.26 81.58) (width 0.7) (layer B.Cu) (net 1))
 (segment (start 90.40502 83.62502) (end 88.36 81.58) (width 0.7) (layer B.Cu) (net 1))
 (segment (start 127.184546 104.874532) (end 125.384546 104.874532) (width 0.7) (layer B.Cu) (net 1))
 (segment (start 90.40502 83.62502) (end 90.42502 83.62502) (width 0.7) (layer B.Cu) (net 1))
 (segment (start 104.885004 84.37499) (end 106.5 85.989986) (width 0.7) (layer B.Cu) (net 1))
 (segment (start 91.17499 84.37499) (end 104.885004 84.37499) (width 0.7) (layer B.Cu) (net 1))
 (segment (start 90.42502 83.62502) (end 91.17499 84.37499) (width 0.7) (layer B.Cu) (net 1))
 (segment (start 125.384546 104.874532) (end 106.5 85.989986) (width 0.7) (layer B.Cu) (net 1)))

